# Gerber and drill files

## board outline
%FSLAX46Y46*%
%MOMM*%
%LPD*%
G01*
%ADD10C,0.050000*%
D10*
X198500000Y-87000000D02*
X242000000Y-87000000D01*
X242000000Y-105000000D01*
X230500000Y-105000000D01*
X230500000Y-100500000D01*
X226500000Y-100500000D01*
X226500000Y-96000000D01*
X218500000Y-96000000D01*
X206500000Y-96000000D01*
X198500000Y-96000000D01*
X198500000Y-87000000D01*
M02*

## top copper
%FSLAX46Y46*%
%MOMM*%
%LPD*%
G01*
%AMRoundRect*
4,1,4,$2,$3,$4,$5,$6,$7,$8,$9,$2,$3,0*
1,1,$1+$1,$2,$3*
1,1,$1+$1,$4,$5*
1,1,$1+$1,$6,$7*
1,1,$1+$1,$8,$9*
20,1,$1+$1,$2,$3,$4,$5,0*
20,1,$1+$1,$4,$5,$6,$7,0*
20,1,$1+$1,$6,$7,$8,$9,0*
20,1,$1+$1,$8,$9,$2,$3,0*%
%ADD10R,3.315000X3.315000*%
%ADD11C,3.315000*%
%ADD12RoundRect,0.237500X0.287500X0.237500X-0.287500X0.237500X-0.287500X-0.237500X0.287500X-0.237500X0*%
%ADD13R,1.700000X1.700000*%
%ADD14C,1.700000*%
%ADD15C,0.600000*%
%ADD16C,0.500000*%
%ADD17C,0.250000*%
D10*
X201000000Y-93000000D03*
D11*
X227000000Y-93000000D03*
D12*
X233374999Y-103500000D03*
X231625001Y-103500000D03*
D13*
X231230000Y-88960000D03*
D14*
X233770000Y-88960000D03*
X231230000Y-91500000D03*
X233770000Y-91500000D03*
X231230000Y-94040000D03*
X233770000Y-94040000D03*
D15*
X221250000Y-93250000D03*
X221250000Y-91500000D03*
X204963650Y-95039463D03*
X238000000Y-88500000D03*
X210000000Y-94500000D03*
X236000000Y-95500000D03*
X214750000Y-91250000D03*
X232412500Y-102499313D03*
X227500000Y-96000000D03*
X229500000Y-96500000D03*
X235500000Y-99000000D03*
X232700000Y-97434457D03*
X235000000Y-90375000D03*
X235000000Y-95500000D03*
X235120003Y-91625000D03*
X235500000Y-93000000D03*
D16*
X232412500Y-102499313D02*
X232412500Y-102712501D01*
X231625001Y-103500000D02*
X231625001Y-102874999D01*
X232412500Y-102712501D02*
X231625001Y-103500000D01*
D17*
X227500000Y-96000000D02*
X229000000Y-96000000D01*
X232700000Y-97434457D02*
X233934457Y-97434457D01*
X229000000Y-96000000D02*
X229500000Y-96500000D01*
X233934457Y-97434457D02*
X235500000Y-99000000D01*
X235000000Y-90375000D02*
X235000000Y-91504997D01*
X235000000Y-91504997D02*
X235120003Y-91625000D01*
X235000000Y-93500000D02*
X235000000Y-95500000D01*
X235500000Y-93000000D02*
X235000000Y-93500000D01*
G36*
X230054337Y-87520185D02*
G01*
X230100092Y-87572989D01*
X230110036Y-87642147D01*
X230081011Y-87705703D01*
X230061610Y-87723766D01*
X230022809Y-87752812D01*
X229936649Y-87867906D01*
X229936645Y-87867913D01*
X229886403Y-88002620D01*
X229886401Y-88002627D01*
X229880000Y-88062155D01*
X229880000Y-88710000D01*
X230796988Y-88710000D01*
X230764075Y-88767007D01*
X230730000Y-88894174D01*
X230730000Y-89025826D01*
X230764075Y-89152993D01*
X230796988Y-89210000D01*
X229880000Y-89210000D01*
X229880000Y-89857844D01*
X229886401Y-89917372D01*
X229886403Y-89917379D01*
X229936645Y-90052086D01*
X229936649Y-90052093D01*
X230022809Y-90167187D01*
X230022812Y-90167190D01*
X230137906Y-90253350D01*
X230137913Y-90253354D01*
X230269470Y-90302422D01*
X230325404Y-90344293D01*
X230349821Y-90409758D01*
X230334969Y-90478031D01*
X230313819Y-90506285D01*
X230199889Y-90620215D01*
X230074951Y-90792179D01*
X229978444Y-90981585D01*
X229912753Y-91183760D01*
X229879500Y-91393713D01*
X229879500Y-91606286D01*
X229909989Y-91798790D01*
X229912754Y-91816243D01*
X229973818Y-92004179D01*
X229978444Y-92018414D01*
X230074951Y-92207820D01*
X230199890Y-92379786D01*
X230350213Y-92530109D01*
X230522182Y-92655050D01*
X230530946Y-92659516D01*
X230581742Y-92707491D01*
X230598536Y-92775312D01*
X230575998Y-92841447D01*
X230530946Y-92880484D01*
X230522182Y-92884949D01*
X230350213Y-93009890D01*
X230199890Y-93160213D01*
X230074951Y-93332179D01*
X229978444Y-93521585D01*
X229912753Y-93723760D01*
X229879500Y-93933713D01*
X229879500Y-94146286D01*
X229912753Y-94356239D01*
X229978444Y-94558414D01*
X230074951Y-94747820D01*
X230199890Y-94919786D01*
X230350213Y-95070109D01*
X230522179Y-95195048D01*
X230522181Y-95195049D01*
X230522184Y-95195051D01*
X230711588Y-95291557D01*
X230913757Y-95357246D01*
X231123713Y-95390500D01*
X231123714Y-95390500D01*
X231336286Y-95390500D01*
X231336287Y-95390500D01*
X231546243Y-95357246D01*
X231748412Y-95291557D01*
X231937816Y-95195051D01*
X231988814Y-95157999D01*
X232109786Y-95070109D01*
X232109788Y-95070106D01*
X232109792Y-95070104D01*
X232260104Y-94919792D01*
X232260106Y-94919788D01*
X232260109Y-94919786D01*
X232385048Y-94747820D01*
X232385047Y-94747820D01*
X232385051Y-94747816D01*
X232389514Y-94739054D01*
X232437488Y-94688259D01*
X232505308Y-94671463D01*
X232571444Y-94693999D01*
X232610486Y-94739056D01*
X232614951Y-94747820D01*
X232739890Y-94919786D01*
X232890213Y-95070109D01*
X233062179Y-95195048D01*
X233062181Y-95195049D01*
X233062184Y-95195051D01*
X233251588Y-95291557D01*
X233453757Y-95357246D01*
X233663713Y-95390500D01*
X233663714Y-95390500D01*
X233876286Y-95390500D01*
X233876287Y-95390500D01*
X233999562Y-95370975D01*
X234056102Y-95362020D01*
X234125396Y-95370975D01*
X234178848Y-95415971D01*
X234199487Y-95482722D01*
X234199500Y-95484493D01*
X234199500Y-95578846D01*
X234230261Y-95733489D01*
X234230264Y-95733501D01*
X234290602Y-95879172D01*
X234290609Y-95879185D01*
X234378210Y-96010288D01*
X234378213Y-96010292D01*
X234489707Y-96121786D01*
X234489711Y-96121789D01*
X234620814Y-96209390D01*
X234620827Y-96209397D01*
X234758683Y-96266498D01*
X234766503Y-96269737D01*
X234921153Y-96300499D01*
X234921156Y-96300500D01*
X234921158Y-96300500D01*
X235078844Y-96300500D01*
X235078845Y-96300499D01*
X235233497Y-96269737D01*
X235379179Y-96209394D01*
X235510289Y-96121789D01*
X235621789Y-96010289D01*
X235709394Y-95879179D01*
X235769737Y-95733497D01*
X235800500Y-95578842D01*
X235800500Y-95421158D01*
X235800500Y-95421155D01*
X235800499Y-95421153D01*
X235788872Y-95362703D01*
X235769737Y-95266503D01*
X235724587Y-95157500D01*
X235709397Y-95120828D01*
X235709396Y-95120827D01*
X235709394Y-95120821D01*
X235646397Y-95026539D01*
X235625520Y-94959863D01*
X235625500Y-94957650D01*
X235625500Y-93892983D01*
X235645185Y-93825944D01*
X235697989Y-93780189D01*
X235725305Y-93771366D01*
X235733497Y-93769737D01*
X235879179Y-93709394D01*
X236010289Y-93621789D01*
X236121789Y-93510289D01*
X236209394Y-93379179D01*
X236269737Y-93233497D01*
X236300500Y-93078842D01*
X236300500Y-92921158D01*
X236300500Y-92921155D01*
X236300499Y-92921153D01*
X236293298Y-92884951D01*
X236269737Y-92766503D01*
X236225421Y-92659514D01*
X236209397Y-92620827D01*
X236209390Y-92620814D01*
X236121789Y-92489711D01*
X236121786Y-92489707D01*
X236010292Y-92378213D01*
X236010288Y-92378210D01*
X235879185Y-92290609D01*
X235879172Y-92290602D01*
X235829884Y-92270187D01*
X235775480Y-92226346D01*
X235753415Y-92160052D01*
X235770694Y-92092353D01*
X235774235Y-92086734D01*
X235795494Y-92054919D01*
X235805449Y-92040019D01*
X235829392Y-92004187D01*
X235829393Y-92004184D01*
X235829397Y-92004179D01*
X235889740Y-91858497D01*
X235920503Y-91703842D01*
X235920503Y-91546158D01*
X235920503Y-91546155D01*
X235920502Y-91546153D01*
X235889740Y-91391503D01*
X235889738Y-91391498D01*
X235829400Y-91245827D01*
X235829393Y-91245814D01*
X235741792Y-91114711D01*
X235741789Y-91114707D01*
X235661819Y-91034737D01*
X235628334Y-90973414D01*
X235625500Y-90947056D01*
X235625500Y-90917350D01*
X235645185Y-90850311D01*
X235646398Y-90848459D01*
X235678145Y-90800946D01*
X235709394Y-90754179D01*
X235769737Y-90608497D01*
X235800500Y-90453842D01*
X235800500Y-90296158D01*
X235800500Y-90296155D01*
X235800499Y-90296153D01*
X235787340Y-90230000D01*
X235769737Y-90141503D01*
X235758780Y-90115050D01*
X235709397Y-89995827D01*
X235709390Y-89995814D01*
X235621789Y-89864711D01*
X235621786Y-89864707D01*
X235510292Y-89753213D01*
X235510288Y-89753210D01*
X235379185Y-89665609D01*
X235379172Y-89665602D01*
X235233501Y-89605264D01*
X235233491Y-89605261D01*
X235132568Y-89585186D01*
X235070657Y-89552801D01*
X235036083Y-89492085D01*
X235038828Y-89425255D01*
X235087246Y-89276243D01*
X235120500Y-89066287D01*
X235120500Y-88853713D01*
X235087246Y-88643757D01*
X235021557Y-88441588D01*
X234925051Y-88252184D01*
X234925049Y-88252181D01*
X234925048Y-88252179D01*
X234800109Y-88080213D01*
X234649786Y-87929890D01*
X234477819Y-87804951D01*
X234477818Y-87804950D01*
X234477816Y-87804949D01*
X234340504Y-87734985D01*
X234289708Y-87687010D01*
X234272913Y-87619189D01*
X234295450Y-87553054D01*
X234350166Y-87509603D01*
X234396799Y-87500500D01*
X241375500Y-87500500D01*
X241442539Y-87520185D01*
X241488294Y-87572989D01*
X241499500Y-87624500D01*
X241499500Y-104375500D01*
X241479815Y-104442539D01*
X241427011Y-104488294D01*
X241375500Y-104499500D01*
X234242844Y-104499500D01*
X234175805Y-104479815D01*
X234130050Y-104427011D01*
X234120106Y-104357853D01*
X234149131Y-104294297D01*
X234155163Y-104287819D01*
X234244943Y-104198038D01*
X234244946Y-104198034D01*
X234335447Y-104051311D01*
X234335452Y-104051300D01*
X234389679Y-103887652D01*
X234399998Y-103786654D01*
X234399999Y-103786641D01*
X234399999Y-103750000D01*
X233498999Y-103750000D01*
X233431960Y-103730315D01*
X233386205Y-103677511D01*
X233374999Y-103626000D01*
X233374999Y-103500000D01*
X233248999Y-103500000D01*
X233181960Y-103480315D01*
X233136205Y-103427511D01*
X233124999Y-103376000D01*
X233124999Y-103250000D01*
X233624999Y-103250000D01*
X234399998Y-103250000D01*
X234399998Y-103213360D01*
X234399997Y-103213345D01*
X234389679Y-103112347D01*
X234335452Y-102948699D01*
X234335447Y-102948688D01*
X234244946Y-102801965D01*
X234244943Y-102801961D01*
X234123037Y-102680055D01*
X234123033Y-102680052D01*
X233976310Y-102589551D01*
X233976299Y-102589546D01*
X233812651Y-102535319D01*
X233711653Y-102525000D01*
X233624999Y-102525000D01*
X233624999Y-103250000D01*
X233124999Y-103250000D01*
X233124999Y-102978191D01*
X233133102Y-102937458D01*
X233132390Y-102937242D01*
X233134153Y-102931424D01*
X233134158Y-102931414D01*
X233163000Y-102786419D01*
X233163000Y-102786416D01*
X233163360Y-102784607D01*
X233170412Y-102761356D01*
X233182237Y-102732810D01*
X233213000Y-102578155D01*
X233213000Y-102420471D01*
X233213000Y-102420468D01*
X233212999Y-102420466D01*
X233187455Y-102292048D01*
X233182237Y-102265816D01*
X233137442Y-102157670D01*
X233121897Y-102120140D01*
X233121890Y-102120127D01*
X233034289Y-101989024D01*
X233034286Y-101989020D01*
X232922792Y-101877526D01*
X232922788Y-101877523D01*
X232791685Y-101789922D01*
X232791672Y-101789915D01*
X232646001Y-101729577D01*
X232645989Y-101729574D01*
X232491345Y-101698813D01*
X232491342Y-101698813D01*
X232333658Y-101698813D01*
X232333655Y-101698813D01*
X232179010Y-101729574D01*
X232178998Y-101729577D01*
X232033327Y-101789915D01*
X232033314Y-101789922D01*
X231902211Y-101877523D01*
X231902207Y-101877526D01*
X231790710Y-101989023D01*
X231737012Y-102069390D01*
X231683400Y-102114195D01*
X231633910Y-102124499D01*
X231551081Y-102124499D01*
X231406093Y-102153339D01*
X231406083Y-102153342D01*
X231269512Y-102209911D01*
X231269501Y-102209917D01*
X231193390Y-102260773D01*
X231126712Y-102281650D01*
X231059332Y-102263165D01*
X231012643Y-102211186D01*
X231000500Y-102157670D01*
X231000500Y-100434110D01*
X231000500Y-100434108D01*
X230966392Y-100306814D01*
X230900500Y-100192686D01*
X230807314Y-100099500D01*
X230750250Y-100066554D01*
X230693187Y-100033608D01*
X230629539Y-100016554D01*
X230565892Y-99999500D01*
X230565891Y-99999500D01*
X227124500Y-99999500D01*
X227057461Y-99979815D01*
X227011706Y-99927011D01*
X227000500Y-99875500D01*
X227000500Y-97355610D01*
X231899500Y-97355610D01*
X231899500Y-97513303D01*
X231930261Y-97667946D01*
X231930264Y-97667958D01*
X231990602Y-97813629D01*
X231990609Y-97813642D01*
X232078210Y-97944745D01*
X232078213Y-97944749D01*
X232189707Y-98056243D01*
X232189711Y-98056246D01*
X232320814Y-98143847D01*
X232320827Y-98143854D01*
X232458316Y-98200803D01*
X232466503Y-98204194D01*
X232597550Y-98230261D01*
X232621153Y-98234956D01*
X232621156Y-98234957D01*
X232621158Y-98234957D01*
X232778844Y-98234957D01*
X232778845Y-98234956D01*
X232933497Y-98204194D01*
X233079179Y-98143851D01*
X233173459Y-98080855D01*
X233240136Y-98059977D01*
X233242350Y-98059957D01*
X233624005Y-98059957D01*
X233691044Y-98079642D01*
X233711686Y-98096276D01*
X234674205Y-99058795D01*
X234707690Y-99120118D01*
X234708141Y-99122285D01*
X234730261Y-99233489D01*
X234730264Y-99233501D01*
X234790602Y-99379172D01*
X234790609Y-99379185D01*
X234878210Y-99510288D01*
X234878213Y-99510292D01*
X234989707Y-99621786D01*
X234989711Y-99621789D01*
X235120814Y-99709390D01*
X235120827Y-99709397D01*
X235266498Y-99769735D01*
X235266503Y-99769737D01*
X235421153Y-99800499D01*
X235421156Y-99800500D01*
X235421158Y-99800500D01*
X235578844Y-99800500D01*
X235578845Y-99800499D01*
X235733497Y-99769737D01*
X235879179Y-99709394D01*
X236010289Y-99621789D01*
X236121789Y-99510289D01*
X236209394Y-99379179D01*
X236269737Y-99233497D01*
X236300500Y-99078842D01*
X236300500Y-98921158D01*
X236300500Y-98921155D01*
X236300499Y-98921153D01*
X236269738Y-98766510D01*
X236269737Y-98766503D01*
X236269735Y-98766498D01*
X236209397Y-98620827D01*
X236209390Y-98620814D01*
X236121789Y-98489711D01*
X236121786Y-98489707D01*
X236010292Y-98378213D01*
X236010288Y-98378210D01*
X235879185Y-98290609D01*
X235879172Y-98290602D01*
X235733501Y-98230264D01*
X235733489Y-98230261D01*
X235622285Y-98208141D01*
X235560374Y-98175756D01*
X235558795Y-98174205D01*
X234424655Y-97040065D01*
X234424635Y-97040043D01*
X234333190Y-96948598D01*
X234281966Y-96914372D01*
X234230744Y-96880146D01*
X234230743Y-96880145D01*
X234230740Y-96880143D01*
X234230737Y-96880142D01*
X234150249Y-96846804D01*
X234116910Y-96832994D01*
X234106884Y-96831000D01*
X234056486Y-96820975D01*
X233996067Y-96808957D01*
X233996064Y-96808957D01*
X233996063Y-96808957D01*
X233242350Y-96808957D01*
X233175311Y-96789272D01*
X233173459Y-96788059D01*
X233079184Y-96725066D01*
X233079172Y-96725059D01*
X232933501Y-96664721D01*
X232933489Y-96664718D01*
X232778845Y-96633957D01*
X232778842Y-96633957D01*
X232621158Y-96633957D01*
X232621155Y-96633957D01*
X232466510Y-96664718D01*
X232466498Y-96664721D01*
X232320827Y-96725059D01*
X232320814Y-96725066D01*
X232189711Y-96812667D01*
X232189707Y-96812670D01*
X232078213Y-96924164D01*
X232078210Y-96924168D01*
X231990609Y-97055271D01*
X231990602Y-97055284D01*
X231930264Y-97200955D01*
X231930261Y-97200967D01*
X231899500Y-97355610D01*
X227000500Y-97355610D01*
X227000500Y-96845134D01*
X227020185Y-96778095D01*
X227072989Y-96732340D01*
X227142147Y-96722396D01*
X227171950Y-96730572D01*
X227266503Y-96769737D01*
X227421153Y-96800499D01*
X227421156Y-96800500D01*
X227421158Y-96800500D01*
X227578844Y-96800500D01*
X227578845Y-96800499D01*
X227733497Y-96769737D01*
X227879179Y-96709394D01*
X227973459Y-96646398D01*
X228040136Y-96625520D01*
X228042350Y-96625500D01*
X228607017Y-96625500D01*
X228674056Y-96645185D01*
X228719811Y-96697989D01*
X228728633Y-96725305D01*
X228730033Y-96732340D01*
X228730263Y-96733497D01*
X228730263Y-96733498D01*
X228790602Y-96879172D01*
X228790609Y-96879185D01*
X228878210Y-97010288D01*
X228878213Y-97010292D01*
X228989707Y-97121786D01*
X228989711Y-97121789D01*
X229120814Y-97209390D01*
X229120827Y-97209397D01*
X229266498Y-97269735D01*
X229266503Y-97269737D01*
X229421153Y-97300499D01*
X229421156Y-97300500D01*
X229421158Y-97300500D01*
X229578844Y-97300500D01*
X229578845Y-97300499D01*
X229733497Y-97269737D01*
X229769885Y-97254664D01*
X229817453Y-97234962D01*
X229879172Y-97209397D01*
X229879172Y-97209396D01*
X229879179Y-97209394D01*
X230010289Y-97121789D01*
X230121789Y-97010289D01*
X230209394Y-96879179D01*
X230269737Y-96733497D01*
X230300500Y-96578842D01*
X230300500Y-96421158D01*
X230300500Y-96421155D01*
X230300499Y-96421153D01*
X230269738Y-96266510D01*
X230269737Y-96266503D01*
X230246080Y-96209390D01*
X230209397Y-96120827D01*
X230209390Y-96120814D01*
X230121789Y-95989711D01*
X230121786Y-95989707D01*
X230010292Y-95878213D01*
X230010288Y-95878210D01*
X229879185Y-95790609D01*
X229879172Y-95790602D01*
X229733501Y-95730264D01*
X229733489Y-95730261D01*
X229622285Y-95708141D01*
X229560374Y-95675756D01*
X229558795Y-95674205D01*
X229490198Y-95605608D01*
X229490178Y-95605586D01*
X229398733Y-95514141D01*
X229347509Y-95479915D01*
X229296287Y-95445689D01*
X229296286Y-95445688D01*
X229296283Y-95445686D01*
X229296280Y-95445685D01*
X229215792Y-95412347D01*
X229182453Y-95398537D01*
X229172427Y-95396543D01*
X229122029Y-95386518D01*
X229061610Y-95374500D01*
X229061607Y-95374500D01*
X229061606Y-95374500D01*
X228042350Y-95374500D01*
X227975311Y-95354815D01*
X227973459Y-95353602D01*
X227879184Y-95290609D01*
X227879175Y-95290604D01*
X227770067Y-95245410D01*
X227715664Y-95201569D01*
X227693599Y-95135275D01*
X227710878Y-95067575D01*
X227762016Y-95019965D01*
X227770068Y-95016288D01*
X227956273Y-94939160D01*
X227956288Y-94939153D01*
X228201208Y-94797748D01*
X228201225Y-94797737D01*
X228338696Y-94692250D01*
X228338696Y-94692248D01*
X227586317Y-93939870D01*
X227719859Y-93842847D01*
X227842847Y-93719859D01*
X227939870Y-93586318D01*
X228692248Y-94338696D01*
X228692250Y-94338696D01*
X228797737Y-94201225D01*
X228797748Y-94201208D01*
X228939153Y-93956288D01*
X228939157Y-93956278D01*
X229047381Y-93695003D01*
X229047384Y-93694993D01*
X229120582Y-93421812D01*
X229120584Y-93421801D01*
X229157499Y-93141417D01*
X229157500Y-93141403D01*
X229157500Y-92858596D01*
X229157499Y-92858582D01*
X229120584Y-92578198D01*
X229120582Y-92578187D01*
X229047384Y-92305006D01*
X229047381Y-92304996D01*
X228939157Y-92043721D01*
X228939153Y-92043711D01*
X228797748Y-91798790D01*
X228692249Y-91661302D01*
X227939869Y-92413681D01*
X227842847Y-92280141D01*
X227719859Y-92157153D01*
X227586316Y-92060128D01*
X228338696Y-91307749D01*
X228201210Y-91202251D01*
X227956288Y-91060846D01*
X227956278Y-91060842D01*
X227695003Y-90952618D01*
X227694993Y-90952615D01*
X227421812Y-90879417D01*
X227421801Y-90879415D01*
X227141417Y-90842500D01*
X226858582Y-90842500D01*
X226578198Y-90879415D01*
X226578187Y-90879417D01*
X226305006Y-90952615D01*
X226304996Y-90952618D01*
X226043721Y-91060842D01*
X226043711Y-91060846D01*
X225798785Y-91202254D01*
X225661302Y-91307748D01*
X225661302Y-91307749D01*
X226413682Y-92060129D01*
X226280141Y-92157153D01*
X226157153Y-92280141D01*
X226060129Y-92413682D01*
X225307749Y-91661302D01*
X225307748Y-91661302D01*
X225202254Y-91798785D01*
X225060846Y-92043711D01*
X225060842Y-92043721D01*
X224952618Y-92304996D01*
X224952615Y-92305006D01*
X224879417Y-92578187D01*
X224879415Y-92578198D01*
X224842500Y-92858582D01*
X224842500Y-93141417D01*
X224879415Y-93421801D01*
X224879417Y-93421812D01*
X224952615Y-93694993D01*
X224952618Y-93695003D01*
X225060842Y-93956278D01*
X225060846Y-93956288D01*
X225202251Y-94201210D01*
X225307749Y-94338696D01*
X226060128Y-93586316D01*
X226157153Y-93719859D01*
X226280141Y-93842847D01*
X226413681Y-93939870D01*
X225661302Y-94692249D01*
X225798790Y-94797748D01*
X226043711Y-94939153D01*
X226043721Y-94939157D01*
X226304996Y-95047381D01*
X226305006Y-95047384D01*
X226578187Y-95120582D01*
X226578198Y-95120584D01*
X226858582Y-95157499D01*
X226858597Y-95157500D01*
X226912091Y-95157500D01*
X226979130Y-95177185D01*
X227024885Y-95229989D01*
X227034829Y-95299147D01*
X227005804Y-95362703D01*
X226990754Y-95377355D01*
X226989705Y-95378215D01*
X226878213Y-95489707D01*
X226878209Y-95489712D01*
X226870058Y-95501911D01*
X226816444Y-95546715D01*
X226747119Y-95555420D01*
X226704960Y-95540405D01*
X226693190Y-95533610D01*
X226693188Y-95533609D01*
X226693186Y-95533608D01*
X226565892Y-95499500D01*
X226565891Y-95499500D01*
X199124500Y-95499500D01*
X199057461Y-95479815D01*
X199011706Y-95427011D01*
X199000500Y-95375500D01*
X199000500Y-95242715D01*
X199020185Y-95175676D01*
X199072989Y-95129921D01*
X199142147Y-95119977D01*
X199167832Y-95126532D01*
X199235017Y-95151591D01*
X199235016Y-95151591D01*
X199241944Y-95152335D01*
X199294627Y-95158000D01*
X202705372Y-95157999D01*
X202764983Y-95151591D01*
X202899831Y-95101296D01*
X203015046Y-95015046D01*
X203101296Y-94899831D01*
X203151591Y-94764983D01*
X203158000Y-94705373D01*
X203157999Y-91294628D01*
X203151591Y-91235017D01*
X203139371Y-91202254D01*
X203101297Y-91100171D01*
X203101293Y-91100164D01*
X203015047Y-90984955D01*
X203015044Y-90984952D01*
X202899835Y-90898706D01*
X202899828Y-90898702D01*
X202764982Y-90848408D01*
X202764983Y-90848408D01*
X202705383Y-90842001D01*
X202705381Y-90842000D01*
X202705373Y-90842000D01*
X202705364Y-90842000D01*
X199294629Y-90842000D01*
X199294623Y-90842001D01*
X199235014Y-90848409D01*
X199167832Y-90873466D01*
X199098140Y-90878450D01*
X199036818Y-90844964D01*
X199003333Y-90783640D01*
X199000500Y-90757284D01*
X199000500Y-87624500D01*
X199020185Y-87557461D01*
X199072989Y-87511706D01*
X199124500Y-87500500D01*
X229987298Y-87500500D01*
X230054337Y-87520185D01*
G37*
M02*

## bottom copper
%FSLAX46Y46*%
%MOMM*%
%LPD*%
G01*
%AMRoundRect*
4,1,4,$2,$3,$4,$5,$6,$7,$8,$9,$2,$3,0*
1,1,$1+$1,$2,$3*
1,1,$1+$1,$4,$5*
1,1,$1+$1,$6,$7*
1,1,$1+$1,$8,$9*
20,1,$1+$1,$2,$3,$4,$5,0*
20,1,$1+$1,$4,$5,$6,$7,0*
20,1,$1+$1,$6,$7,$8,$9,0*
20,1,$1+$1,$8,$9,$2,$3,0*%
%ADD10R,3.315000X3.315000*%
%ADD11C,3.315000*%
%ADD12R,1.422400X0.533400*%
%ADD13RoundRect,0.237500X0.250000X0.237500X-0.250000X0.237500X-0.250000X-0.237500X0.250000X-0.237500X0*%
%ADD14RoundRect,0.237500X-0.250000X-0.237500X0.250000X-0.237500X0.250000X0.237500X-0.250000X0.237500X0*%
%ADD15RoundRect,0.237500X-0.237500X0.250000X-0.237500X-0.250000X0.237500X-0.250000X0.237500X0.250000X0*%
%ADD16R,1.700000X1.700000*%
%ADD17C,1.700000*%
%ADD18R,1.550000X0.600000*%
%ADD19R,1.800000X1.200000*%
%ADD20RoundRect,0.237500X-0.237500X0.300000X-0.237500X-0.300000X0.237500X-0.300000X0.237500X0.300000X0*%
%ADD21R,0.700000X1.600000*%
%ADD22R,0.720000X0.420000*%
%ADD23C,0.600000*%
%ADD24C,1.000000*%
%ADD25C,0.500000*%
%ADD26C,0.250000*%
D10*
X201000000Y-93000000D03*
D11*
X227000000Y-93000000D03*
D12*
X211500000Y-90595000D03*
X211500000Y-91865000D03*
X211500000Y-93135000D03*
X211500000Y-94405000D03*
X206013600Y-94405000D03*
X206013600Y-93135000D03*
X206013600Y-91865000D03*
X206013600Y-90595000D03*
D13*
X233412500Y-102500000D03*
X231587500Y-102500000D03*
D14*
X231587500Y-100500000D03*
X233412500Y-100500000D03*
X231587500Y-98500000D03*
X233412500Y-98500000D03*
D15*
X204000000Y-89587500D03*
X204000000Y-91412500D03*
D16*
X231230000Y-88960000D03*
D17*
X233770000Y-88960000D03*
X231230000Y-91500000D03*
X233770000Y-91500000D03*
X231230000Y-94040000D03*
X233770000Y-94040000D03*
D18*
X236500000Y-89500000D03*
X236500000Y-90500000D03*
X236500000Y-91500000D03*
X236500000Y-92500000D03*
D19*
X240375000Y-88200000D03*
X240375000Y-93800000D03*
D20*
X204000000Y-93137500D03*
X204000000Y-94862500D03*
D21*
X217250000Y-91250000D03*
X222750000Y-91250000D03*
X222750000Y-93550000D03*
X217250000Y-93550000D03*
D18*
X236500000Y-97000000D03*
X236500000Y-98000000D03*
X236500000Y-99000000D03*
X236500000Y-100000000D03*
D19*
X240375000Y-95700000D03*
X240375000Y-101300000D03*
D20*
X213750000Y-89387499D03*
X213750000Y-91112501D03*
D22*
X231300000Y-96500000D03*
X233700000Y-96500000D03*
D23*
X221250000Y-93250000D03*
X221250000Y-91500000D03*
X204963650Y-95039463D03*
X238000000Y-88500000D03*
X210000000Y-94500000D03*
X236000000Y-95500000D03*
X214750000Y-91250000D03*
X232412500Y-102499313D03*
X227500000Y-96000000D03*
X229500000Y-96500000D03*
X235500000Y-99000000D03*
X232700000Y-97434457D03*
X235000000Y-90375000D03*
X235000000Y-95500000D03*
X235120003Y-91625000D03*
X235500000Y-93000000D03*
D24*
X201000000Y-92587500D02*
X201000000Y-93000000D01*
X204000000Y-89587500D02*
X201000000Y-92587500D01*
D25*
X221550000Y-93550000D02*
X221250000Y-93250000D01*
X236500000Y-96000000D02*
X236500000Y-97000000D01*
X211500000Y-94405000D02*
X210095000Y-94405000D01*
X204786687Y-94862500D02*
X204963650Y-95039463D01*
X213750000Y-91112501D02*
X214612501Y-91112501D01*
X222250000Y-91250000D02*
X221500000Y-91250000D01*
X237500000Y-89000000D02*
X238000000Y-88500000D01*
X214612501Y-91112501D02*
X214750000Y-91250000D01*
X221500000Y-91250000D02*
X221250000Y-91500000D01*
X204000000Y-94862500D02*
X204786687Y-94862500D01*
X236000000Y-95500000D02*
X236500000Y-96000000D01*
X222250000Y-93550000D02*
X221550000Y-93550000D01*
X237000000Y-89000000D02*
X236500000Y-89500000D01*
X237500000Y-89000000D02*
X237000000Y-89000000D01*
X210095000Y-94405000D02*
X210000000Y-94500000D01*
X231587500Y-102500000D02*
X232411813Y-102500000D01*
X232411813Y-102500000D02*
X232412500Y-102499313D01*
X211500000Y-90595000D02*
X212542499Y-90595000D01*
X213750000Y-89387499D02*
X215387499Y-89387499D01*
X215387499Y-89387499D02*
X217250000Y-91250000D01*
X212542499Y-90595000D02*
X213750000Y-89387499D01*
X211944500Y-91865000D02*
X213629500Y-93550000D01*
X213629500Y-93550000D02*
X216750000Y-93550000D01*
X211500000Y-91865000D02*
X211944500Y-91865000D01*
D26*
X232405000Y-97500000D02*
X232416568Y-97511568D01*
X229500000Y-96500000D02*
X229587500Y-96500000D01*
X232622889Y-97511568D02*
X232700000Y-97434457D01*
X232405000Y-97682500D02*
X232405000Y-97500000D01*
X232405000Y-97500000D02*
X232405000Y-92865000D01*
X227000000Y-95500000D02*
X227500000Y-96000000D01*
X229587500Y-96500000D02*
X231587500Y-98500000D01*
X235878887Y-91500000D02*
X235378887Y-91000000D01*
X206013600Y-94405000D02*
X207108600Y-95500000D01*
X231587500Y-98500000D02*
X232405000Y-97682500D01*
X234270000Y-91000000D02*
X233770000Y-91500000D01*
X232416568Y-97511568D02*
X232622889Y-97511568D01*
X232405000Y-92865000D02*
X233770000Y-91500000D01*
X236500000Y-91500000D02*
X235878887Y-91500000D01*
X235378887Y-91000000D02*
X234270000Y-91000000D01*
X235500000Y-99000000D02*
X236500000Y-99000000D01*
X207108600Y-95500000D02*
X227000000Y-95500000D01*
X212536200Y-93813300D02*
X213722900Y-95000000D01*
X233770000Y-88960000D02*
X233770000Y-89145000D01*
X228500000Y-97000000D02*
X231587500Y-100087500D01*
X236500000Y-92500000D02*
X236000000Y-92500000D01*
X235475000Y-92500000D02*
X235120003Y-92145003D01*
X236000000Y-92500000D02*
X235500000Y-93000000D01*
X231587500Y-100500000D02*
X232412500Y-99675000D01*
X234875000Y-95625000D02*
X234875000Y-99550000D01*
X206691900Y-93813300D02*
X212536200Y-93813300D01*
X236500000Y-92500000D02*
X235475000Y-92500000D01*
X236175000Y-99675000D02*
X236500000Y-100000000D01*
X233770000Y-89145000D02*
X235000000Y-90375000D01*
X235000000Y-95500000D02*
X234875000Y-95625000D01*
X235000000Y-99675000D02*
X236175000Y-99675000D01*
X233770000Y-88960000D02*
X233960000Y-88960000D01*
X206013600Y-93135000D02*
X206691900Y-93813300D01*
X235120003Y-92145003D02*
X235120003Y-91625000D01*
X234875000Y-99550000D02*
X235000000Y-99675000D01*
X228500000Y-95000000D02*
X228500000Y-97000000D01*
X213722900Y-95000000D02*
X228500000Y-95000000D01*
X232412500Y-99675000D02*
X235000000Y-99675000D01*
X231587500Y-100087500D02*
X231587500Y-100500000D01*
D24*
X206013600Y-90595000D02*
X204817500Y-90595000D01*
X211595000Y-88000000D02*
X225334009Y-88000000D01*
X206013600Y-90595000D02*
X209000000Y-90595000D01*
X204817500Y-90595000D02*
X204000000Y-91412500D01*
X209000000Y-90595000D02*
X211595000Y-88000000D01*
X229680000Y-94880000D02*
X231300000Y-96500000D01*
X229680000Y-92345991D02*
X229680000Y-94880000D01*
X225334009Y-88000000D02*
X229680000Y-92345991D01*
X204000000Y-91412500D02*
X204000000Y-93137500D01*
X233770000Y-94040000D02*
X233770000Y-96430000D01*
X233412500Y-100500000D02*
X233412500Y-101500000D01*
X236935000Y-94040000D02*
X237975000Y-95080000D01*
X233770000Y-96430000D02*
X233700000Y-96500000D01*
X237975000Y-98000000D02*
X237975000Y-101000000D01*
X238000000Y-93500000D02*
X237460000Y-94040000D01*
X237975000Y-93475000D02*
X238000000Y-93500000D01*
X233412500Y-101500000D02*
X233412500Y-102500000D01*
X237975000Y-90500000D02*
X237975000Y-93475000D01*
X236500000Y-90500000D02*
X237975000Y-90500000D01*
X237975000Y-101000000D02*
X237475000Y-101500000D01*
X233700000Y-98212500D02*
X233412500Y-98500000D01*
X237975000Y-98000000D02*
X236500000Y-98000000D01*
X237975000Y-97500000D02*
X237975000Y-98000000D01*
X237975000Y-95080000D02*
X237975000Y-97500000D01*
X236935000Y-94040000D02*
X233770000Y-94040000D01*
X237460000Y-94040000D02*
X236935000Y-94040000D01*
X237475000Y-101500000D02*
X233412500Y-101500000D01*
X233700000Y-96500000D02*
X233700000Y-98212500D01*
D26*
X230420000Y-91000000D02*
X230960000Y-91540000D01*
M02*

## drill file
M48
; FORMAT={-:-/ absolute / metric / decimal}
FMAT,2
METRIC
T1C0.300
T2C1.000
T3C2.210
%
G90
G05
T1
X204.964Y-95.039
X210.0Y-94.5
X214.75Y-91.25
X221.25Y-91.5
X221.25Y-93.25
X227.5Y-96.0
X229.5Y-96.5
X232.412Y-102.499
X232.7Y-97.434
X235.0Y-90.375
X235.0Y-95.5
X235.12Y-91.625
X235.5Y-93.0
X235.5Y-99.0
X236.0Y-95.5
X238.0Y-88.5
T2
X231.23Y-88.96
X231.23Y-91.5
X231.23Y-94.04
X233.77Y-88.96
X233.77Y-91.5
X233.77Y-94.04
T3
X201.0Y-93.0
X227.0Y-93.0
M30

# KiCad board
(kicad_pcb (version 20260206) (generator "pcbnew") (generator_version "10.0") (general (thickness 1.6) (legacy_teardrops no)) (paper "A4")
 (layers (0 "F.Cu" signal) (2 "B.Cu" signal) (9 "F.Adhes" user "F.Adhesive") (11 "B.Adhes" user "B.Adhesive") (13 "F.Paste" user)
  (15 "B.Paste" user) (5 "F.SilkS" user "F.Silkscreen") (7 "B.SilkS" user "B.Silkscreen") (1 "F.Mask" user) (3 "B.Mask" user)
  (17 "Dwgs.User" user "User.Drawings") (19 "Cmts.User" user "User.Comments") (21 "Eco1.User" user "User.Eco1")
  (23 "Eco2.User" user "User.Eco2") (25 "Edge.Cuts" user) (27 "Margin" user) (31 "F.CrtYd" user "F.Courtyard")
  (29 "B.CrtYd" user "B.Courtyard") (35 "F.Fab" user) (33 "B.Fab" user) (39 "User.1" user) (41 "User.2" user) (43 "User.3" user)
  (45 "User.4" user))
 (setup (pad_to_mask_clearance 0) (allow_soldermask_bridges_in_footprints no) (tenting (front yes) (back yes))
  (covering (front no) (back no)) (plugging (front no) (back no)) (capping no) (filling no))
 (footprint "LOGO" (layer "F.Cu") (at 239.5 89.5 90)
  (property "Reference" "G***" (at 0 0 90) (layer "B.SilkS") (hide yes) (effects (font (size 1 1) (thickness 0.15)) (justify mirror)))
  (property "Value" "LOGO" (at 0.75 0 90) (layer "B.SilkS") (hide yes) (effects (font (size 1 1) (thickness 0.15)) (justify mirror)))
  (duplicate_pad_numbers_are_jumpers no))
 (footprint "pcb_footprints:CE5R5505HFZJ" (layer "F.Cu") (at 201 93 180)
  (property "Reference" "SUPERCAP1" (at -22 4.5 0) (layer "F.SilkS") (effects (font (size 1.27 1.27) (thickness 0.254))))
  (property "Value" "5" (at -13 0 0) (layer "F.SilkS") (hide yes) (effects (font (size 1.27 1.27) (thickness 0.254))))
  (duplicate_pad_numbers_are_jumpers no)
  (pad "1" thru_hole rect (at 0 0 180) (size 3.315 3.315) (drill 2.21) (layers "*.Cu" "*.Mask") (remove_unused_layers no)
   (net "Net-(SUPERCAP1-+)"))
  (pad "2" thru_hole circle (at -26 0 180) (size 3.315 3.315) (drill 2.21) (layers "*.Cu" "*.Mask") (remove_unused_layers no) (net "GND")))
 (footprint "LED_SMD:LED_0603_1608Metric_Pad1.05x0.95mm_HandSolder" (layer "F.Cu") (at 232.5 103.5 180)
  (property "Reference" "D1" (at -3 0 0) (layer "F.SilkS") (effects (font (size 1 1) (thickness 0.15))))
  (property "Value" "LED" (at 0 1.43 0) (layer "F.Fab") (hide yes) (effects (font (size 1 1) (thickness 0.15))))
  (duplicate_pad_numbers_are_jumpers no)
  (pad "1" smd roundrect (at -0.874999 0 180) (size 1.05 0.95) (layers "F.Cu" "F.Mask" "F.Paste") (roundrect_rratio 0.25) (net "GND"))
  (pad "2" smd roundrect (at 0.874999 0 180) (size 1.05 0.95) (layers "F.Cu" "F.Mask" "F.Paste") (roundrect_rratio 0.25) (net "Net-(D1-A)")))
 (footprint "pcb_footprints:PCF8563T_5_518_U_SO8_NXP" (layer "B.Cu") (at 208.7568 92.5 180)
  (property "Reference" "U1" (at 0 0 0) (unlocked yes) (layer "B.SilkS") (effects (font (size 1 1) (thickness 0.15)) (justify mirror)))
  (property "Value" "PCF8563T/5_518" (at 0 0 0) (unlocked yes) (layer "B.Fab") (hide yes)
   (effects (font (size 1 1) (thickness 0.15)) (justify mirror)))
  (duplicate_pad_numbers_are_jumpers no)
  (pad "1" smd rect (at -2.7432 1.905 180) (size 1.4224 0.5334) (layers "B.Cu" "B.Mask" "B.Paste") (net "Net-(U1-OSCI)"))
  (pad "2" smd rect (at -2.7432 0.635 180) (size 1.4224 0.5334) (layers "B.Cu" "B.Mask" "B.Paste") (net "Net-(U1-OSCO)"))
  (pad "3" smd rect (at -2.7432 -0.635 180) (size 1.4224 0.5334) (layers "B.Cu" "B.Mask" "B.Paste") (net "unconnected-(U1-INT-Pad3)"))
  (pad "4" smd rect (at -2.7432 -1.905 180) (size 1.4224 0.5334) (layers "B.Cu" "B.Mask" "B.Paste") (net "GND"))
  (pad "5" smd rect (at 2.7432 -1.905 180) (size 1.4224 0.5334) (layers "B.Cu" "B.Mask" "B.Paste") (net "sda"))
  (pad "6" smd rect (at 2.7432 -0.635 180) (size 1.4224 0.5334) (layers "B.Cu" "B.Mask" "B.Paste") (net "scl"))
  (pad "7" smd rect (at 2.7432 0.635 180) (size 1.4224 0.5334) (layers "B.Cu" "B.Mask" "B.Paste") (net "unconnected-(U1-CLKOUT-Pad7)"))
  (pad "8" smd rect (at 2.7432 1.905 180) (size 1.4224 0.5334) (layers "B.Cu" "B.Mask" "B.Paste") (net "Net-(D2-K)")))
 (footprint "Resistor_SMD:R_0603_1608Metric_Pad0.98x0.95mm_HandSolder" (layer "B.Cu") (at 232.5 102.5 180)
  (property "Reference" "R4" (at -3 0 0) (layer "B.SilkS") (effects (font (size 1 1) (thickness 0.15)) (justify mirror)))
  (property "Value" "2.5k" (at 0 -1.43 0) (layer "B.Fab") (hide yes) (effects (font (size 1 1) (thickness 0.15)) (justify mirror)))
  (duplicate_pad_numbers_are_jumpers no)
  (pad "1" smd roundrect (at -0.9125 0 180) (size 0.975 0.95) (layers "B.Cu" "B.Mask" "B.Paste") (roundrect_rratio 0.25) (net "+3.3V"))
  (pad "2" smd roundrect (at 0.9125 0 180) (size 0.975 0.95) (layers "B.Cu" "B.Mask" "B.Paste") (roundrect_rratio 0.25) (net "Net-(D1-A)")))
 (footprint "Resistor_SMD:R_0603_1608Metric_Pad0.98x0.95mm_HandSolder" (layer "B.Cu") (at 232.5 100.5)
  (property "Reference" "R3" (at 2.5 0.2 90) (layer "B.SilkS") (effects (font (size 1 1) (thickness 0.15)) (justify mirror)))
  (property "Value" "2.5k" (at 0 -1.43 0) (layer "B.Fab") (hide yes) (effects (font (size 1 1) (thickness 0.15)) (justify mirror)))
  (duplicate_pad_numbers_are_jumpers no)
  (pad "1" smd roundrect (at -0.9125 0) (size 0.975 0.95) (layers "B.Cu" "B.Mask" "B.Paste") (roundrect_rratio 0.25) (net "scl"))
  (pad "2" smd roundrect (at 0.9125 0) (size 0.975 0.95) (layers "B.Cu" "B.Mask" "B.Paste") (roundrect_rratio 0.25) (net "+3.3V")))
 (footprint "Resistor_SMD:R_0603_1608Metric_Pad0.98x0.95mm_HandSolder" (layer "B.Cu") (at 232.5 98.5)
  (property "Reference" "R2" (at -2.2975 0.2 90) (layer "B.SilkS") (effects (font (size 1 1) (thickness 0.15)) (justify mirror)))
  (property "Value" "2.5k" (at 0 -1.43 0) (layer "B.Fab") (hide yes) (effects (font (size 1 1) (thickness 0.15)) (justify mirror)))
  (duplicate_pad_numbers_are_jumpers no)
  (pad "1" smd roundrect (at -0.9125 0) (size 0.975 0.95) (layers "B.Cu" "B.Mask" "B.Paste") (roundrect_rratio 0.25) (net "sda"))
  (pad "2" smd roundrect (at 0.9125 0) (size 0.975 0.95) (layers "B.Cu" "B.Mask" "B.Paste") (roundrect_rratio 0.25) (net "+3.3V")))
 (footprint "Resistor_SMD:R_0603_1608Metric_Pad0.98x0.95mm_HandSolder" (layer "B.Cu") (at 204 90.5 -90)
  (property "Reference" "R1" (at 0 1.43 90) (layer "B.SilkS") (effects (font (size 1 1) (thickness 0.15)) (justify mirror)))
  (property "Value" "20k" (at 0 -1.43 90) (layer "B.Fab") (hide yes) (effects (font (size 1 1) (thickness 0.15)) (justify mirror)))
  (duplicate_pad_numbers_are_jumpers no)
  (pad "1" smd roundrect (at -0.9125 0 270) (size 0.975 0.95) (layers "B.Cu" "B.Mask" "B.Paste") (roundrect_rratio 0.25)
   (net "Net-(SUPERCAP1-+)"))
  (pad "2" smd roundrect (at 0.9125 0 270) (size 0.975 0.95) (layers "B.Cu" "B.Mask" "B.Paste") (roundrect_rratio 0.25) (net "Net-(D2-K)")))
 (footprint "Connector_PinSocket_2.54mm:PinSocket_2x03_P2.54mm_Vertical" (layer "B.Cu") (at 231.23 88.96 180)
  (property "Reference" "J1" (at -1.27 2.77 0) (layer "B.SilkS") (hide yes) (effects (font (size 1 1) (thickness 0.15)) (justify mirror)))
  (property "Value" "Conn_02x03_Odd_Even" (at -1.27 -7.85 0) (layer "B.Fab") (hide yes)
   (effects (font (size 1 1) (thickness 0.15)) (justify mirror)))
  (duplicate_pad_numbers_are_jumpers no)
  (pad "1" thru_hole rect (at 0 0 180) (size 1.7 1.7) (drill 1) (layers "*.Cu" "*.Mask") (remove_unused_layers no) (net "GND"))
  (pad "2" thru_hole circle (at -2.54 0 180) (size 1.7 1.7) (drill 1) (layers "*.Cu" "*.Mask") (remove_unused_layers no) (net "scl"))
  (pad "3" thru_hole circle (at 0 -2.54 180) (size 1.7 1.7) (drill 1) (layers "*.Cu" "*.Mask") (remove_unused_layers no)
   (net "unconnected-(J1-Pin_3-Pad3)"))
  (pad "4" thru_hole circle (at -2.54 -2.54 180) (size 1.7 1.7) (drill 1) (layers "*.Cu" "*.Mask") (remove_unused_layers no) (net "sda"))
  (pad "5" thru_hole circle (at 0 -5.08 180) (size 1.7 1.7) (drill 1) (layers "*.Cu" "*.Mask") (remove_unused_layers no)
   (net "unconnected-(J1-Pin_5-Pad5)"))
  (pad "6" thru_hole circle (at -2.54 -5.08 180) (size 1.7 1.7) (drill 1) (layers "*.Cu" "*.Mask") (remove_unused_layers no) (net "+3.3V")))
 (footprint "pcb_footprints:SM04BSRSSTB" (layer "B.Cu") (at 238.787 91 -90)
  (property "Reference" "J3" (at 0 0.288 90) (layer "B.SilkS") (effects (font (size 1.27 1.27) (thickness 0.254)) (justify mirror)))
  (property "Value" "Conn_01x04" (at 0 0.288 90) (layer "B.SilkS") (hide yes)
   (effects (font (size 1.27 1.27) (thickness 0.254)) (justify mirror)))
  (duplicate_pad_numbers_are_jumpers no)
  (pad "1" smd rect (at -1.5 2.287 270) (size 0.6 1.55) (layers "B.Cu" "B.Mask" "B.Paste") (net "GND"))
  (pad "2" smd rect (at -0.5 2.287 270) (size 0.6 1.55) (layers "B.Cu" "B.Mask" "B.Paste") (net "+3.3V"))
  (pad "3" smd rect (at 0.5 2.287 270) (size 0.6 1.55) (layers "B.Cu" "B.Mask" "B.Paste") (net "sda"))
  (pad "4" smd rect (at 1.5 2.287 270) (size 0.6 1.55) (layers "B.Cu" "B.Mask" "B.Paste") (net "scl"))
  (pad "MP1" smd rect (at -2.8 -1.588 270) (size 1.2 1.8) (layers "B.Cu" "B.Mask" "B.Paste"))
  (pad "MP2" smd rect (at 2.8 -1.588 270) (size 1.2 1.8) (layers "B.Cu" "B.Mask" "B.Paste")))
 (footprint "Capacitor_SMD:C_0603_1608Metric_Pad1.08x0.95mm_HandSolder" (layer "B.Cu") (at 204 94 -90)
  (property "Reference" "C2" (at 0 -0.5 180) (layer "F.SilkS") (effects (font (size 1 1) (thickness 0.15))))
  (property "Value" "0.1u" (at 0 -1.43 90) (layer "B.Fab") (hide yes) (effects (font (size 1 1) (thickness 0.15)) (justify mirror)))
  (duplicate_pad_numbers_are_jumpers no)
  (pad "1" smd roundrect (at -0.8625 0 270) (size 1.075 0.95) (layers "B.Cu" "B.Mask" "B.Paste") (roundrect_rratio 0.25) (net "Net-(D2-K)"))
  (pad "2" smd roundrect (at 0.8625 0 270) (size 1.075 0.95) (layers "B.Cu" "B.Mask" "B.Paste") (roundrect_rratio 0.25) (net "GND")))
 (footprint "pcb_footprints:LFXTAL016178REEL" (layer "B.Cu") (at 220 92.4)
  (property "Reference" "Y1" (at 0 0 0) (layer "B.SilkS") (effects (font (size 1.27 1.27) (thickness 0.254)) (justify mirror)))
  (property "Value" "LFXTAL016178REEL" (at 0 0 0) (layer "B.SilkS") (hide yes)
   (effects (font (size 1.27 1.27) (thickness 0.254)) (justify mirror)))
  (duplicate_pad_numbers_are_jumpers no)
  (pad "1" smd rect (at -2.75 -1.15) (size 0.7 1.6) (layers "B.Cu" "B.Mask" "B.Paste") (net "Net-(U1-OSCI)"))
  (pad "2" smd rect (at 2.75 -1.15) (size 0.7 1.6) (layers "B.Cu" "B.Mask" "B.Paste") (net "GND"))
  (pad "3" smd rect (at 2.75 1.15) (size 0.7 1.6) (layers "B.Cu" "B.Mask" "B.Paste") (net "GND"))
  (pad "4" smd rect (at -2.75 1.15) (size 0.7 1.6) (layers "B.Cu" "B.Mask" "B.Paste") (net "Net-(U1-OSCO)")))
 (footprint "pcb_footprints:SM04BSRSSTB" (layer "B.Cu") (at 238.787 98.5 -90)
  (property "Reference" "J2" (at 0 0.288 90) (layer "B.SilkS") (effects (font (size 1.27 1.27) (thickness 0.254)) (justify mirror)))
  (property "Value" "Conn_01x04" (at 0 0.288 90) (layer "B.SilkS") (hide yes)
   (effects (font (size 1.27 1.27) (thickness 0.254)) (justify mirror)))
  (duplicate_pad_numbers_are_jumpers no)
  (pad "1" smd rect (at -1.5 2.287 270) (size 0.6 1.55) (layers "B.Cu" "B.Mask" "B.Paste") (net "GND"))
  (pad "2" smd rect (at -0.5 2.287 270) (size 0.6 1.55) (layers "B.Cu" "B.Mask" "B.Paste") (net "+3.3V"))
  (pad "3" smd rect (at 0.5 2.287 270) (size 0.6 1.55) (layers "B.Cu" "B.Mask" "B.Paste") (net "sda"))
  (pad "4" smd rect (at 1.5 2.287 270) (size 0.6 1.55) (layers "B.Cu" "B.Mask" "B.Paste") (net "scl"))
  (pad "MP1" smd rect (at -2.8 -1.588 270) (size 1.2 1.8) (layers "B.Cu" "B.Mask" "B.Paste"))
  (pad "MP2" smd rect (at 2.8 -1.588 270) (size 1.2 1.8) (layers "B.Cu" "B.Mask" "B.Paste")))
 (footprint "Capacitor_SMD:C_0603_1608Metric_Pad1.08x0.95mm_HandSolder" (layer "B.Cu") (at 213.75 90.25 -90)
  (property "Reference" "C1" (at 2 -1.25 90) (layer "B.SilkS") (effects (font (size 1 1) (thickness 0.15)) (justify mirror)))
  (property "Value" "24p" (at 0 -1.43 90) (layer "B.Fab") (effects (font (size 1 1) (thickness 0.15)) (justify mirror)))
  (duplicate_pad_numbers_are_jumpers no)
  (pad "1" smd roundrect (at -0.862501 0 270) (size 1.075 0.95) (layers "B.Cu" "B.Mask" "B.Paste") (roundrect_rratio 0.25)
   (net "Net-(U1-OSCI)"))
  (pad "2" smd roundrect (at 0.862501 0 270) (size 1.075 0.95) (layers "B.Cu" "B.Mask" "B.Paste") (roundrect_rratio 0.25) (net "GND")))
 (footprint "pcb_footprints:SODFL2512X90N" (layer "B.Cu") (at 232.5 96.5)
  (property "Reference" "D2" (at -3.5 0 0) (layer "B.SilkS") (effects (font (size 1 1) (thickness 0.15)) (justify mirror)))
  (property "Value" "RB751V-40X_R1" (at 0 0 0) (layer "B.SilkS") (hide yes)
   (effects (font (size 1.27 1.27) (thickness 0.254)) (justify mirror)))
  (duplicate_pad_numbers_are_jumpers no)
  (pad "1" smd rect (at -1.2 0 270) (size 0.42 0.72) (layers "B.Cu" "B.Mask" "B.Paste") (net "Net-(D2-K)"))
  (pad "2" smd rect (at 1.2 0 270) (size 0.42 0.72) (layers "B.Cu" "B.Mask" "B.Paste") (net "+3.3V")))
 (gr_poly
  (pts (xy 198.5 87) (xy 242 87) (xy 242 105) (xy 230.5 105) (xy 230.5 100.5) (xy 226.5 100.5) (xy 226.5 96) (xy 218.5 96) (xy 206.5 96)
   (xy 198.5 96))
  (stroke (width 0.05) (type solid)) (fill no) (layer "Edge.Cuts"))
 (segment (start 201 92.5875) (end 201 93) (width 1) (layer "B.Cu") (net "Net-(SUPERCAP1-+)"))
 (segment (start 204 89.5875) (end 201 92.5875) (width 1) (layer "B.Cu") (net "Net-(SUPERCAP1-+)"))
 (via (at 221.25 93.25) (size 0.6) (drill 0.3) (layers "F.Cu" "B.Cu") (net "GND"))
 (via (at 221.25 91.5) (size 0.6) (drill 0.3) (layers "F.Cu" "B.Cu") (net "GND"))
 (via (at 204.96365 95.039463) (size 0.6) (drill 0.3) (layers "F.Cu" "B.Cu") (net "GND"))
 (via (at 238 88.5) (size 0.6) (drill 0.3) (layers "F.Cu" "B.Cu") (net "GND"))
 (via (at 210 94.5) (size 0.6) (drill 0.3) (layers "F.Cu" "B.Cu") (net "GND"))
 (via (at 236 95.5) (size 0.6) (drill 0.3) (layers "F.Cu" "B.Cu") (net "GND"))
 (via (at 214.75 91.25) (size 0.6) (drill 0.3) (layers "F.Cu" "B.Cu") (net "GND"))
 (segment (start 221.55 93.55) (end 221.25 93.25) (width 0.5) (layer "B.Cu") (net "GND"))
 (segment (start 236.5 96) (end 236.5 97) (width 0.5) (layer "B.Cu") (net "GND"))
 (segment (start 211.5 94.405) (end 210.095 94.405) (width 0.5) (layer "B.Cu") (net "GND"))
 (segment (start 204.786687 94.8625) (end 204.96365 95.039463) (width 0.5) (layer "B.Cu") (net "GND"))
 (segment (start 213.75 91.112501) (end 214.612501 91.112501) (width 0.5) (layer "B.Cu") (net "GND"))
 (segment (start 222.25 91.25) (end 221.5 91.25) (width 0.5) (layer "B.Cu") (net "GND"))
 (segment (start 237.5 89) (end 238 88.5) (width 0.5) (layer "B.Cu") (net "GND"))
 (segment (start 214.612501 91.112501) (end 214.75 91.25) (width 0.5) (layer "B.Cu") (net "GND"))
 (segment (start 221.5 91.25) (end 221.25 91.5) (width 0.5) (layer "B.Cu") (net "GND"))
 (segment (start 204 94.8625) (end 204.786687 94.8625) (width 0.5) (layer "B.Cu") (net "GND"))
 (segment (start 236 95.5) (end 236.5 96) (width 0.5) (layer "B.Cu") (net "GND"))
 (segment (start 222.25 93.55) (end 221.55 93.55) (width 0.5) (layer "B.Cu") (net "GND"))
 (segment (start 237 89) (end 236.5 89.5) (width 0.5) (layer "B.Cu") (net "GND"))
 (segment (start 237.5 89) (end 237 89) (width 0.5) (layer "B.Cu") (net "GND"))
 (segment (start 210.095 94.405) (end 210 94.5) (width 0.5) (layer "B.Cu") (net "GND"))
 (segment (start 232.4125 102.499313) (end 232.4125 102.712501) (width 0.5) (layer "F.Cu") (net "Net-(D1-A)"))
 (segment (start 231.625001 103.5) (end 231.625001 102.874999) (width 0.5) (layer "F.Cu") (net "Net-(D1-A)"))
 (segment (start 232.4125 102.712501) (end 231.625001 103.5) (width 0.5) (layer "F.Cu") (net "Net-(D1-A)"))
 (via (at 232.4125 102.499313) (size 0.6) (drill 0.3) (layers "F.Cu" "B.Cu") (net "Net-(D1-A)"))
 (segment (start 231.5875 102.5) (end 232.411813 102.5) (width 0.5) (layer "B.Cu") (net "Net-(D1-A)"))
 (segment (start 232.411813 102.5) (end 232.4125 102.499313) (width 0.5) (layer "B.Cu") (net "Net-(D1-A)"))
 (segment (start 211.5 90.595) (end 212.542499 90.595) (width 0.5) (layer "B.Cu") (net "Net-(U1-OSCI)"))
 (segment (start 213.75 89.387499) (end 215.387499 89.387499) (width 0.5) (layer "B.Cu") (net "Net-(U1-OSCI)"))
 (segment (start 215.387499 89.387499) (end 217.25 91.25) (width 0.5) (layer "B.Cu") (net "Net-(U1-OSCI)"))
 (segment (start 212.542499 90.595) (end 213.75 89.387499) (width 0.5) (layer "B.Cu") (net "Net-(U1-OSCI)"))
 (segment (start 211.9445 91.865) (end 213.6295 93.55) (width 0.5) (layer "B.Cu") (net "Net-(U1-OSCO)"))
 (segment (start 213.6295 93.55) (end 216.75 93.55) (width 0.5) (layer "B.Cu") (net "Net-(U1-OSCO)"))
 (segment (start 211.5 91.865) (end 211.9445 91.865) (width 0.5) (layer "B.Cu") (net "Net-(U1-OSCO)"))
 (segment (start 227.5 96) (end 229 96) (width 0.25) (layer "F.Cu") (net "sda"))
 (segment (start 232.7 97.434457) (end 233.934457 97.434457) (width 0.25) (layer "F.Cu") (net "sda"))
 (segment (start 229 96) (end 229.5 96.5) (width 0.25) (layer "F.Cu") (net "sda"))
 (segment (start 233.934457 97.434457) (end 235.5 99) (width 0.25) (layer "F.Cu") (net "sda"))
 (via (at 227.5 96) (size 0.6) (drill 0.3) (layers "F.Cu" "B.Cu") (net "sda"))
 (via (at 229.5 96.5) (size 0.6) (drill 0.3) (layers "F.Cu" "B.Cu") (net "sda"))
 (via (at 235.5 99) (size 0.6) (drill 0.3) (layers "F.Cu" "B.Cu") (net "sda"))
 (via (at 232.7 97.434457) (size 0.6) (drill 0.3) (layers "F.Cu" "B.Cu") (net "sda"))
 (segment (start 232.405 97.5) (end 232.416568 97.511568) (width 0.25) (layer "B.Cu") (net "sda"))
 (segment (start 229.5 96.5) (end 229.5875 96.5) (width 0.25) (layer "B.Cu") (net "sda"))
 (segment (start 232.622889 97.511568) (end 232.7 97.434457) (width 0.25) (layer "B.Cu") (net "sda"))
 (segment (start 232.405 97.6825) (end 232.405 97.5) (width 0.25) (layer "B.Cu") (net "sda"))
 (segment (start 232.405 97.5) (end 232.405 92.865) (width 0.25) (layer "B.Cu") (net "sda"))
 (segment (start 227 95.5) (end 227.5 96) (width 0.25) (layer "B.Cu") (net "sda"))
 (segment (start 229.5875 96.5) (end 231.5875 98.5) (width 0.25) (layer "B.Cu") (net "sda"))
 (segment (start 235.878887 91.5) (end 235.378887 91) (width 0.25) (layer "B.Cu") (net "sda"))
 (segment (start 206.0136 94.405) (end 207.1086 95.5) (width 0.25) (layer "B.Cu") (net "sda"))
 (segment (start 231.5875 98.5) (end 232.405 97.6825) (width 0.25) (layer "B.Cu") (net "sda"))
 (segment (start 234.27 91) (end 233.77 91.5) (width 0.25) (layer "B.Cu") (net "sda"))
 (segment (start 232.416568 97.511568) (end 232.622889 97.511568) (width 0.25) (layer "B.Cu") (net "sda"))
 (segment (start 232.405 92.865) (end 233.77 91.5) (width 0.25) (layer "B.Cu") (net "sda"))
 (segment (start 236.5 91.5) (end 235.878887 91.5) (width 0.25) (layer "B.Cu") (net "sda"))
 (segment (start 235.378887 91) (end 234.27 91) (width 0.25) (layer "B.Cu") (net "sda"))
 (segment (start 235.5 99) (end 236.5 99) (width 0.25) (layer "B.Cu") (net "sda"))
 (segment (start 207.1086 95.5) (end 227 95.5) (width 0.25) (layer "B.Cu") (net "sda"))
 (segment (start 235 90.375) (end 235 91.504997) (width 0.25) (layer "F.Cu") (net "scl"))
 (segment (start 235 91.504997) (end 235.120003 91.625) (width 0.25) (layer "F.Cu") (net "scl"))
 (segment (start 235 93.5) (end 235 95.5) (width 0.25) (layer "F.Cu") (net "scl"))
 (segment (start 235.5 93) (end 235 93.5) (width 0.25) (layer "F.Cu") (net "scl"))
 (via (at 235 90.375) (size 0.6) (drill 0.3) (layers "F.Cu" "B.Cu") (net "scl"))
 (via (at 235 95.5) (size 0.6) (drill 0.3) (layers "F.Cu" "B.Cu") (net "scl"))
 (via (at 235.120003 91.625) (size 0.6) (drill 0.3) (layers "F.Cu" "B.Cu") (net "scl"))
 (via (at 235.5 93) (size 0.6) (drill 0.3) (layers "F.Cu" "B.Cu") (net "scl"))
 (segment (start 212.5362 93.8133) (end 213.7229 95) (width 0.25) (layer "B.Cu") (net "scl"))
 (segment (start 233.77 88.96) (end 233.77 89.145) (width 0.25) (layer "B.Cu") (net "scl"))
 (segment (start 228.5 97) (end 231.5875 100.0875) (width 0.25) (layer "B.Cu") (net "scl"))
 (segment (start 236.5 92.5) (end 236 92.5) (width 0.25) (layer "B.Cu") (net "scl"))
 (segment (start 235.475 92.5) (end 235.120003 92.145003) (width 0.25) (layer "B.Cu") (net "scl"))
 (segment (start 236 92.5) (end 235.5 93) (width 0.25) (layer "B.Cu") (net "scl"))
 (segment (start 231.5875 100.5) (end 232.4125 99.675) (width 0.25) (layer "B.Cu") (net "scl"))
 (segment (start 234.875 95.625) (end 234.875 99.55) (width 0.25) (layer "B.Cu") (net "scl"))
 (segment (start 206.6919 93.8133) (end 212.5362 93.8133) (width 0.25) (layer "B.Cu") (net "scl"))
 (segment (start 236.5 92.5) (end 235.475 92.5) (width 0.25) (layer "B.Cu") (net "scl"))
 (segment (start 236.175 99.675) (end 236.5 100) (width 0.25) (layer "B.Cu") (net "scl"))
 (segment (start 233.77 89.145) (end 235 90.375) (width 0.25) (layer "B.Cu") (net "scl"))
 (segment (start 235 95.5) (end 234.875 95.625) (width 0.25) (layer "B.Cu") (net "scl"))
 (segment (start 235 99.675) (end 236.175 99.675) (width 0.25) (layer "B.Cu") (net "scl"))
 (segment (start 233.77 88.96) (end 233.96 88.96) (width 0.25) (layer "B.Cu") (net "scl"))
 (segment (start 206.0136 93.135) (end 206.6919 93.8133) (width 0.25) (layer "B.Cu") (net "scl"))
 (segment (start 235.120003 92.145003) (end 235.120003 91.625) (width 0.25) (layer "B.Cu") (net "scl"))
 (segment (start 234.875 99.55) (end 235 99.675) (width 0.25) (layer "B.Cu") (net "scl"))
 (segment (start 228.5 95) (end 228.5 97) (width 0.25) (layer "B.Cu") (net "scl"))
 (segment (start 213.7229 95) (end 228.5 95) (width 0.25) (layer "B.Cu") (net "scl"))
 (segment (start 232.4125 99.675) (end 235 99.675) (width 0.25) (layer "B.Cu") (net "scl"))
 (segment (start 231.5875 100.0875) (end 231.5875 100.5) (width 0.25) (layer "B.Cu") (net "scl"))
 (segment (start 206.0136 90.595) (end 204.8175 90.595) (width 1) (layer "B.Cu") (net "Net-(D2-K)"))
 (segment (start 211.595 88) (end 225.334009 88) (width 1) (layer "B.Cu") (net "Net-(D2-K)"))
 (segment (start 206.0136 90.595) (end 209 90.595) (width 1) (layer "B.Cu") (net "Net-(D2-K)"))
 (segment (start 204.8175 90.595) (end 204 91.4125) (width 1) (layer "B.Cu") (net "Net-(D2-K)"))
 (segment (start 209 90.595) (end 211.595 88) (width 1) (layer "B.Cu") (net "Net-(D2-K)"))
 (segment (start 229.68 94.88) (end 231.3 96.5) (width 1) (layer "B.Cu") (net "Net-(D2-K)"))
 (segment (start 229.68 92.345991) (end 229.68 94.88) (width 1) (layer "B.Cu") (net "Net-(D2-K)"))
 (segment (start 225.334009 88) (end 229.68 92.345991) (width 1) (layer "B.Cu") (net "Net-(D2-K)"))
 (segment (start 204 91.4125) (end 204 93.1375) (width 1) (layer "B.Cu") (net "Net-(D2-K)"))
 (segment (start 233.77 94.04) (end 233.77 96.43) (width 1) (layer "B.Cu") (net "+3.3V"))
 (segment (start 233.4125 100.5) (end 233.4125 101.5) (width 1) (layer "B.Cu") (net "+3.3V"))
 (segment (start 236.935 94.04) (end 237.975 95.08) (width 1) (layer "B.Cu") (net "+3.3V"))
 (segment (start 233.77 96.43) (end 233.7 96.5) (width 1) (layer "B.Cu") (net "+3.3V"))
 (segment (start 237.975 98) (end 237.975 101) (width 1) (layer "B.Cu") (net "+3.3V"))
 (segment (start 238 93.5) (end 237.46 94.04) (width 1) (layer "B.Cu") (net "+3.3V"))
 (segment (start 237.975 93.475) (end 238 93.5) (width 1) (layer "B.Cu") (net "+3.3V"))
 (segment (start 233.4125 101.5) (end 233.4125 102.5) (width 1) (layer "B.Cu") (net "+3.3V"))
 (segment (start 237.975 90.5) (end 237.975 93.475) (width 1) (layer "B.Cu") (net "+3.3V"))
 (segment (start 236.5 90.5) (end 237.975 90.5) (width 1) (layer "B.Cu") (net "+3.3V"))
 (segment (start 237.975 101) (end 237.475 101.5) (width 1) (layer "B.Cu") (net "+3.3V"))
 (segment (start 233.7 98.2125) (end 233.4125 98.5) (width 1) (layer "B.Cu") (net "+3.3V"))
 (segment (start 237.975 98) (end 236.5 98) (width 1) (layer "B.Cu") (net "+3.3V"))
 (segment (start 237.975 97.5) (end 237.975 98) (width 1) (layer "B.Cu") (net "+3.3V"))
 (segment (start 237.975 95.08) (end 237.975 97.5) (width 1) (layer "B.Cu") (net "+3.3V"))
 (segment (start 236.935 94.04) (end 233.77 94.04) (width 1) (layer "B.Cu") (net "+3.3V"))
 (segment (start 237.46 94.04) (end 236.935 94.04) (width 1) (layer "B.Cu") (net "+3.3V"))
 (segment (start 237.475 101.5) (end 233.4125 101.5) (width 1) (layer "B.Cu") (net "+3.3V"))
 (segment (start 233.7 96.5) (end 233.7 98.2125) (width 1) (layer "B.Cu") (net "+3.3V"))
 (segment (start 230.42 91) (end 230.96 91.54) (width 0.25) (layer "B.Cu") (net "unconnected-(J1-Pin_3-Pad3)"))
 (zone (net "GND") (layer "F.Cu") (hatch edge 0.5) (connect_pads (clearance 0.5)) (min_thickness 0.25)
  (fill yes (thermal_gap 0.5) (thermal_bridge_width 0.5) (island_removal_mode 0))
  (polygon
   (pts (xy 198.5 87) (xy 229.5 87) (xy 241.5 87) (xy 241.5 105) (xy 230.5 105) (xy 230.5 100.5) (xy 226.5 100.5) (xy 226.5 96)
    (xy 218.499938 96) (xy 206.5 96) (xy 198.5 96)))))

